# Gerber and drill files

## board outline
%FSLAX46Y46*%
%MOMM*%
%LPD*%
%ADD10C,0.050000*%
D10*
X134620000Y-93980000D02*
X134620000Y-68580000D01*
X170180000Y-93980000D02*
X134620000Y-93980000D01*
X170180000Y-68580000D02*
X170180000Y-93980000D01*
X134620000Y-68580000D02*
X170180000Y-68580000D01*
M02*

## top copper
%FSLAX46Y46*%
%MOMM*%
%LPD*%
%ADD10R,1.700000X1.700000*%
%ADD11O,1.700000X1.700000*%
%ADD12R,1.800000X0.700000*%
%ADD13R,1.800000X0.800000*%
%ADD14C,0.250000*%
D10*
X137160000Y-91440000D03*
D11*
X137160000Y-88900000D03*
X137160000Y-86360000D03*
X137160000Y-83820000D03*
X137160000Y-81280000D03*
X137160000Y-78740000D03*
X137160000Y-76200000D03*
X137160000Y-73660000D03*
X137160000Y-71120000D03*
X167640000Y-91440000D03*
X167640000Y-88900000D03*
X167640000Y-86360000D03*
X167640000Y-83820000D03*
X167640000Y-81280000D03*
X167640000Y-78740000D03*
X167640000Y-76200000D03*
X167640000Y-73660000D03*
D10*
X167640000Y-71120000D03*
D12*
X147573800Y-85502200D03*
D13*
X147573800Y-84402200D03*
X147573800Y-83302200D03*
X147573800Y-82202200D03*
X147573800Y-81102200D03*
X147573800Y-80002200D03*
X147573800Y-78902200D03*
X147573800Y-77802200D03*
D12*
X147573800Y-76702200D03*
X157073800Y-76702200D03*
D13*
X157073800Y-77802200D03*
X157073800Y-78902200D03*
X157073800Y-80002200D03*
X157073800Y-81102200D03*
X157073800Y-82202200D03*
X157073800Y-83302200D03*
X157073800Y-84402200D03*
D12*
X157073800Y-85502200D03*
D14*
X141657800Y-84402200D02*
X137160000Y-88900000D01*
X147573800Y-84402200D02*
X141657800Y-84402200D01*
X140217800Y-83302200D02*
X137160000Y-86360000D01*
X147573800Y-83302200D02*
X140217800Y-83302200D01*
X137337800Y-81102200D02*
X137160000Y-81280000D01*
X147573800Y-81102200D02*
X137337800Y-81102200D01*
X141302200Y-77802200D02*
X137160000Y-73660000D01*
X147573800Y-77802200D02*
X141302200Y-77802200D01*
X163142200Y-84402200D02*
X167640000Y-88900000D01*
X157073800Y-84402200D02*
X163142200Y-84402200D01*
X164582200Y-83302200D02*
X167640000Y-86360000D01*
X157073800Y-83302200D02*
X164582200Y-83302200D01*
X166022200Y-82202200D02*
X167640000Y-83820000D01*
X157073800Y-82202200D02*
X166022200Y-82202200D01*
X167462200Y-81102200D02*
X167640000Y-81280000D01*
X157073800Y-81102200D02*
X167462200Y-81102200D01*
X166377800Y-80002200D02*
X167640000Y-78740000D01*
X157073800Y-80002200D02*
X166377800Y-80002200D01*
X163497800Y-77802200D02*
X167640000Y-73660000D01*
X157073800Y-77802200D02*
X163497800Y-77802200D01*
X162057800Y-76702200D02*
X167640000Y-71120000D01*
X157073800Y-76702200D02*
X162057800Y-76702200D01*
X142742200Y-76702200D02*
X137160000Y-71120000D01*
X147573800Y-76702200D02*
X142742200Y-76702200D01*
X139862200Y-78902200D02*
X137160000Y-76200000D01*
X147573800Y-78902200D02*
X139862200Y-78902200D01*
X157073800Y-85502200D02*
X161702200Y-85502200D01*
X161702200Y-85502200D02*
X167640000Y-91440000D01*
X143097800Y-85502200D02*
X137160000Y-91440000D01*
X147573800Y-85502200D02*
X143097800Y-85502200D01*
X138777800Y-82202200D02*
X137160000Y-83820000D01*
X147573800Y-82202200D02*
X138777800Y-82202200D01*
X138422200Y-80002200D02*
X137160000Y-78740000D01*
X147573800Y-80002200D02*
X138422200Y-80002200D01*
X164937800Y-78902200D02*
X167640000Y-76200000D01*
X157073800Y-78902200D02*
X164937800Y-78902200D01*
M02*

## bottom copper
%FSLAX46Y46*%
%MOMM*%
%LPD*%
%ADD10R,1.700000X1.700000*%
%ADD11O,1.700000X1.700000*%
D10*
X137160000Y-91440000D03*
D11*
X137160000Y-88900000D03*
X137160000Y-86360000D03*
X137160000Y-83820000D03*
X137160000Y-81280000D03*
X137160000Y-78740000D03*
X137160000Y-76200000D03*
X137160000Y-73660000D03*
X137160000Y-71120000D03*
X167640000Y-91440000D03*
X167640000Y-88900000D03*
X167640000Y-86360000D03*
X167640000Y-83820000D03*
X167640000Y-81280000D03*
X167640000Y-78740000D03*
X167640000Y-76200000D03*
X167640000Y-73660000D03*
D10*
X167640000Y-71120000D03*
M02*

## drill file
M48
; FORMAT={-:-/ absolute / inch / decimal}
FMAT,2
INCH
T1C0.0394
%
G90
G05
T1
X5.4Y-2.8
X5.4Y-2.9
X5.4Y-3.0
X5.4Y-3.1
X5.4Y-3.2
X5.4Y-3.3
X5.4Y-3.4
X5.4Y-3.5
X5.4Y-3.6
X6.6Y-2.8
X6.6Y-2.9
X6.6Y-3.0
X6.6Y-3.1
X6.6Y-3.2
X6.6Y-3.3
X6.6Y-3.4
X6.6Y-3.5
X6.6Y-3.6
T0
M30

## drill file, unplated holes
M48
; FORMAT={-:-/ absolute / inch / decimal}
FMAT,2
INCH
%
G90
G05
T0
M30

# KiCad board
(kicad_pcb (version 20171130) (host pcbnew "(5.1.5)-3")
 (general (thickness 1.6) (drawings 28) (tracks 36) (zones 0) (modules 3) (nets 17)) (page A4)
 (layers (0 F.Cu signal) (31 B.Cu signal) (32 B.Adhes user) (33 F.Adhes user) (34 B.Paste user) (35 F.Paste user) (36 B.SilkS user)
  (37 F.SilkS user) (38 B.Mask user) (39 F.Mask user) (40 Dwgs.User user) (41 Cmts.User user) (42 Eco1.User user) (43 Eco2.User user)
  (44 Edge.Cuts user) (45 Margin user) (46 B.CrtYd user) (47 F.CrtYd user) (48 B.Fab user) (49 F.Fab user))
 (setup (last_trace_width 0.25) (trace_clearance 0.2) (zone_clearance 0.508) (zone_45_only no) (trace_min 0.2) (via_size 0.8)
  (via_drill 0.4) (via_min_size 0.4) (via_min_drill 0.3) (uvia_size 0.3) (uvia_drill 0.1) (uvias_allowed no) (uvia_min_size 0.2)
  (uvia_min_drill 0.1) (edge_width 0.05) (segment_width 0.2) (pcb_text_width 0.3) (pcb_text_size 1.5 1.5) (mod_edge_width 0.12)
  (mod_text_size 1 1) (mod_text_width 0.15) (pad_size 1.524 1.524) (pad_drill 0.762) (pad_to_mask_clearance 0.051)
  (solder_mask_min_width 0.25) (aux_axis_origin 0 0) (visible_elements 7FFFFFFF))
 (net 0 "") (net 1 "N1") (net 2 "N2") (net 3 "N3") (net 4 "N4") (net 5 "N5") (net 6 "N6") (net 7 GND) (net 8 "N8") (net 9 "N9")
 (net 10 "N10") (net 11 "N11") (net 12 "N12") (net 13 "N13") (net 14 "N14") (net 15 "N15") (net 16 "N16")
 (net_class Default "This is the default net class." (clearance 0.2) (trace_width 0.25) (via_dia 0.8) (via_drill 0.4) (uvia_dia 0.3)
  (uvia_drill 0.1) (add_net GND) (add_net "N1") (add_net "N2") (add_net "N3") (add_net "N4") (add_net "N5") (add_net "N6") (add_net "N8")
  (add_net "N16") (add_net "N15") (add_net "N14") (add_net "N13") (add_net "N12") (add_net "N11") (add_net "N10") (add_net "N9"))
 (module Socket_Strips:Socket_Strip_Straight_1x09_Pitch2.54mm (layer F.Cu) (at 137.16 91.44 180)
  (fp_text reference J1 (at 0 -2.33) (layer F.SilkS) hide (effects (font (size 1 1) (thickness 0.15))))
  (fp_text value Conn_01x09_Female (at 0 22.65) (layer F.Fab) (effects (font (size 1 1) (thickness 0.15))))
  (pad 1 thru_hole rect (at 0 0 180) (size 1.7 1.7) (drill 1) (layers *.Cu *.Mask) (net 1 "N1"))
  (pad 2 thru_hole oval (at 0 2.54 180) (size 1.7 1.7) (drill 1) (layers *.Cu *.Mask) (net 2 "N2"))
  (pad 3 thru_hole oval (at 0 5.08 180) (size 1.7 1.7) (drill 1) (layers *.Cu *.Mask) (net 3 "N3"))
  (pad 4 thru_hole oval (at 0 7.62 180) (size 1.7 1.7) (drill 1) (layers *.Cu *.Mask) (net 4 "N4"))
  (pad 5 thru_hole oval (at 0 10.16 180) (size 1.7 1.7) (drill 1) (layers *.Cu *.Mask) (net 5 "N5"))
  (pad 6 thru_hole oval (at 0 12.7 180) (size 1.7 1.7) (drill 1) (layers *.Cu *.Mask) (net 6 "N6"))
  (pad 7 thru_hole oval (at 0 15.24 180) (size 1.7 1.7) (drill 1) (layers *.Cu *.Mask) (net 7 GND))
  (pad 8 thru_hole oval (at 0 17.78 180) (size 1.7 1.7) (drill 1) (layers *.Cu *.Mask) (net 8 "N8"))
  (pad 9 thru_hole oval (at 0 20.32 180) (size 1.7 1.7) (drill 1) (layers *.Cu *.Mask) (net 7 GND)))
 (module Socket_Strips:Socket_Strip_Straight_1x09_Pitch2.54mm (layer F.Cu) (at 167.64 71.12)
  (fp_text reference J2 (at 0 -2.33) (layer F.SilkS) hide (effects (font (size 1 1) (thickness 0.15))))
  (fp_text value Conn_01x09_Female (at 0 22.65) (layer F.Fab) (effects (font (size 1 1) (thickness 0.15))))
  (pad 9 thru_hole oval (at 0 20.32) (size 1.7 1.7) (drill 1) (layers *.Cu *.Mask) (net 7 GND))
  (pad 8 thru_hole oval (at 0 17.78) (size 1.7 1.7) (drill 1) (layers *.Cu *.Mask) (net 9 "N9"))
  (pad 7 thru_hole oval (at 0 15.24) (size 1.7 1.7) (drill 1) (layers *.Cu *.Mask) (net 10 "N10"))
  (pad 6 thru_hole oval (at 0 12.7) (size 1.7 1.7) (drill 1) (layers *.Cu *.Mask) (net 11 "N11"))
  (pad 5 thru_hole oval (at 0 10.16) (size 1.7 1.7) (drill 1) (layers *.Cu *.Mask) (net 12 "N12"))
  (pad 4 thru_hole oval (at 0 7.62) (size 1.7 1.7) (drill 1) (layers *.Cu *.Mask) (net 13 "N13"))
  (pad 3 thru_hole oval (at 0 5.08) (size 1.7 1.7) (drill 1) (layers *.Cu *.Mask) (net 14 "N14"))
  (pad 2 thru_hole oval (at 0 2.54) (size 1.7 1.7) (drill 1) (layers *.Cu *.Mask) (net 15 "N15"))
  (pad 1 thru_hole rect (at 0 0) (size 1.7 1.7) (drill 1) (layers *.Cu *.Mask) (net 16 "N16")))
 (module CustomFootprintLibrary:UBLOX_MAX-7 (layer F.Cu) (at 152.4 81.28)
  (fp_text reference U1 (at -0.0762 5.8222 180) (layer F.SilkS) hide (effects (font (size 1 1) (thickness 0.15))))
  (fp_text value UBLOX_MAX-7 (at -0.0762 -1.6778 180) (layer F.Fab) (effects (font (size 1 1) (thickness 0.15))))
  (pad 18 smd rect (at -4.8262 4.2222 180) (size 1.8 0.7) (layers F.Cu F.Paste F.Mask) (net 1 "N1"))
  (pad 17 smd rect (at -4.8262 3.1222 180) (size 1.8 0.8) (layers F.Cu F.Paste F.Mask) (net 2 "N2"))
  (pad 16 smd rect (at -4.8262 2.0222 180) (size 1.8 0.8) (layers F.Cu F.Paste F.Mask) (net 3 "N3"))
  (pad 15 smd rect (at -4.8262 0.9222 180) (size 1.8 0.8) (layers F.Cu F.Paste F.Mask) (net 4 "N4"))
  (pad 14 smd rect (at -4.8262 -0.1778 180) (size 1.8 0.8) (layers F.Cu F.Paste F.Mask) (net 5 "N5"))
  (pad 13 smd rect (at -4.8262 -1.2778 180) (size 1.8 0.8) (layers F.Cu F.Paste F.Mask) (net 6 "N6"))
  (pad 12 smd rect (at -4.8262 -2.3778 180) (size 1.8 0.8) (layers F.Cu F.Paste F.Mask) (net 7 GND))
  (pad 11 smd rect (at -4.8262 -3.4778 180) (size 1.8 0.8) (layers F.Cu F.Paste F.Mask) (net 8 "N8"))
  (pad 10 smd rect (at -4.8262 -4.5778 180) (size 1.8 0.7) (layers F.Cu F.Paste F.Mask) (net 7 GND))
  (pad 9 smd rect (at 4.6738 -4.5778 180) (size 1.8 0.7) (layers F.Cu F.Paste F.Mask) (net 16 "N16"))
  (pad 8 smd rect (at 4.6738 -3.4778 180) (size 1.8 0.8) (layers F.Cu F.Paste F.Mask) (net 15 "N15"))
  (pad 7 smd rect (at 4.6738 -2.3778 180) (size 1.8 0.8) (layers F.Cu F.Paste F.Mask) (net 14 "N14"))
  (pad 6 smd rect (at 4.6738 -1.2778 180) (size 1.8 0.8) (layers F.Cu F.Paste F.Mask) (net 13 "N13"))
  (pad 5 smd rect (at 4.6738 -0.1778 180) (size 1.8 0.8) (layers F.Cu F.Paste F.Mask) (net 12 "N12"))
  (pad 4 smd rect (at 4.6738 0.9222 180) (size 1.8 0.8) (layers F.Cu F.Paste F.Mask) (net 11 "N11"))
  (pad 3 smd rect (at 4.6738 2.0222 180) (size 1.8 0.8) (layers F.Cu F.Paste F.Mask) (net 10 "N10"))
  (pad 2 smd rect (at 4.6738 3.1222 180) (size 1.8 0.8) (layers F.Cu F.Paste F.Mask) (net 9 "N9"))
  (pad 1 smd rect (at 4.6738 4.2222 180) (size 1.8 0.7) (layers F.Cu F.Paste F.Mask) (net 7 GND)))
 (gr_line (start 134.62 93.98) (end 134.62 68.58) (layer Edge.Cuts) (width 0.05))
 (gr_line (start 170.18 93.98) (end 134.62 93.98) (layer Edge.Cuts) (width 0.05))
 (gr_line (start 170.18 68.58) (end 170.18 93.98) (layer Edge.Cuts) (width 0.05))
 (gr_line (start 134.62 68.58) (end 170.18 68.58) (layer Edge.Cuts) (width 0.05))
 (segment (start 141.6578 84.4022) (end 137.16 88.9) (width 0.25) (layer F.Cu) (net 2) (status 20))
 (segment (start 147.5738 84.4022) (end 141.6578 84.4022) (width 0.25) (layer F.Cu) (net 2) (status 10))
 (segment (start 140.2178 83.3022) (end 137.16 86.36) (width 0.25) (layer F.Cu) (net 3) (status 20))
 (segment (start 147.5738 83.3022) (end 140.2178 83.3022) (width 0.25) (layer F.Cu) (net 3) (status 10))
 (segment (start 137.3378 81.1022) (end 137.16 81.28) (width 0.25) (layer F.Cu) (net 5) (status 30))
 (segment (start 147.5738 81.1022) (end 137.3378 81.1022) (width 0.25) (layer F.Cu) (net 5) (status 30))
 (segment (start 141.3022 77.8022) (end 137.16 73.66) (width 0.25) (layer F.Cu) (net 8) (status 20))
 (segment (start 147.5738 77.8022) (end 141.3022 77.8022) (width 0.25) (layer F.Cu) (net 8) (status 10))
 (segment (start 163.1422 84.4022) (end 167.64 88.9) (width 0.25) (layer F.Cu) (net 9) (status 20))
 (segment (start 157.0738 84.4022) (end 163.1422 84.4022) (width 0.25) (layer F.Cu) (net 9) (status 10))
 (segment (start 164.5822 83.3022) (end 167.64 86.36) (width 0.25) (layer F.Cu) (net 10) (status 20))
 (segment (start 157.0738 83.3022) (end 164.5822 83.3022) (width 0.25) (layer F.Cu) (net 10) (status 10))
 (segment (start 166.0222 82.2022) (end 167.64 83.82) (width 0.25) (layer F.Cu) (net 11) (status 20))
 (segment (start 157.0738 82.2022) (end 166.0222 82.2022) (width 0.25) (layer F.Cu) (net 11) (status 10))
 (segment (start 167.4622 81.1022) (end 167.64 81.28) (width 0.25) (layer F.Cu) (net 12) (status 30))
 (segment (start 157.0738 81.1022) (end 167.4622 81.1022) (width 0.25) (layer F.Cu) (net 12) (status 30))
 (segment (start 166.3778 80.0022) (end 167.64 78.74) (width 0.25) (layer F.Cu) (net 13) (status 20))
 (segment (start 157.0738 80.0022) (end 166.3778 80.0022) (width 0.25) (layer F.Cu) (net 13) (status 10))
 (segment (start 163.4978 77.8022) (end 167.64 73.66) (width 0.25) (layer F.Cu) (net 15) (status 20))
 (segment (start 157.0738 77.8022) (end 163.4978 77.8022) (width 0.25) (layer F.Cu) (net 15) (status 10))
 (segment (start 162.0578 76.7022) (end 167.64 71.12) (width 0.25) (layer F.Cu) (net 16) (status 20))
 (segment (start 157.0738 76.7022) (end 162.0578 76.7022) (width 0.25) (layer F.Cu) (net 16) (status 10))
 (segment (start 142.7422 76.7022) (end 137.16 71.12) (width 0.25) (layer F.Cu) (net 7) (status 20))
 (segment (start 147.5738 76.7022) (end 142.7422 76.7022) (width 0.25) (layer F.Cu) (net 7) (status 10))
 (segment (start 139.8622 78.9022) (end 137.16 76.2) (width 0.25) (layer F.Cu) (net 7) (status 20))
 (segment (start 147.5738 78.9022) (end 139.8622 78.9022) (width 0.25) (layer F.Cu) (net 7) (status 10))
 (segment (start 157.0738 85.5022) (end 161.7022 85.5022) (width 0.25) (layer F.Cu) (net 7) (status 10))
 (segment (start 161.7022 85.5022) (end 167.64 91.44) (width 0.25) (layer F.Cu) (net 7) (status 20))
 (segment (start 143.0978 85.5022) (end 137.16 91.44) (width 0.25) (layer F.Cu) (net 1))
 (segment (start 147.5738 85.5022) (end 143.0978 85.5022) (width 0.25) (layer F.Cu) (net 1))
 (segment (start 138.7778 82.2022) (end 137.16 83.82) (width 0.25) (layer F.Cu) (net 4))
 (segment (start 147.5738 82.2022) (end 138.7778 82.2022) (width 0.25) (layer F.Cu) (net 4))
 (segment (start 138.4222 80.0022) (end 137.16 78.74) (width 0.25) (layer F.Cu) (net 6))
 (segment (start 147.5738 80.0022) (end 138.4222 80.0022) (width 0.25) (layer F.Cu) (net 6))
 (segment (start 164.9378 78.9022) (end 167.64 76.2) (width 0.25) (layer F.Cu) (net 14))
 (segment (start 157.0738 78.9022) (end 164.9378 78.9022) (width 0.25) (layer F.Cu) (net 14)))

